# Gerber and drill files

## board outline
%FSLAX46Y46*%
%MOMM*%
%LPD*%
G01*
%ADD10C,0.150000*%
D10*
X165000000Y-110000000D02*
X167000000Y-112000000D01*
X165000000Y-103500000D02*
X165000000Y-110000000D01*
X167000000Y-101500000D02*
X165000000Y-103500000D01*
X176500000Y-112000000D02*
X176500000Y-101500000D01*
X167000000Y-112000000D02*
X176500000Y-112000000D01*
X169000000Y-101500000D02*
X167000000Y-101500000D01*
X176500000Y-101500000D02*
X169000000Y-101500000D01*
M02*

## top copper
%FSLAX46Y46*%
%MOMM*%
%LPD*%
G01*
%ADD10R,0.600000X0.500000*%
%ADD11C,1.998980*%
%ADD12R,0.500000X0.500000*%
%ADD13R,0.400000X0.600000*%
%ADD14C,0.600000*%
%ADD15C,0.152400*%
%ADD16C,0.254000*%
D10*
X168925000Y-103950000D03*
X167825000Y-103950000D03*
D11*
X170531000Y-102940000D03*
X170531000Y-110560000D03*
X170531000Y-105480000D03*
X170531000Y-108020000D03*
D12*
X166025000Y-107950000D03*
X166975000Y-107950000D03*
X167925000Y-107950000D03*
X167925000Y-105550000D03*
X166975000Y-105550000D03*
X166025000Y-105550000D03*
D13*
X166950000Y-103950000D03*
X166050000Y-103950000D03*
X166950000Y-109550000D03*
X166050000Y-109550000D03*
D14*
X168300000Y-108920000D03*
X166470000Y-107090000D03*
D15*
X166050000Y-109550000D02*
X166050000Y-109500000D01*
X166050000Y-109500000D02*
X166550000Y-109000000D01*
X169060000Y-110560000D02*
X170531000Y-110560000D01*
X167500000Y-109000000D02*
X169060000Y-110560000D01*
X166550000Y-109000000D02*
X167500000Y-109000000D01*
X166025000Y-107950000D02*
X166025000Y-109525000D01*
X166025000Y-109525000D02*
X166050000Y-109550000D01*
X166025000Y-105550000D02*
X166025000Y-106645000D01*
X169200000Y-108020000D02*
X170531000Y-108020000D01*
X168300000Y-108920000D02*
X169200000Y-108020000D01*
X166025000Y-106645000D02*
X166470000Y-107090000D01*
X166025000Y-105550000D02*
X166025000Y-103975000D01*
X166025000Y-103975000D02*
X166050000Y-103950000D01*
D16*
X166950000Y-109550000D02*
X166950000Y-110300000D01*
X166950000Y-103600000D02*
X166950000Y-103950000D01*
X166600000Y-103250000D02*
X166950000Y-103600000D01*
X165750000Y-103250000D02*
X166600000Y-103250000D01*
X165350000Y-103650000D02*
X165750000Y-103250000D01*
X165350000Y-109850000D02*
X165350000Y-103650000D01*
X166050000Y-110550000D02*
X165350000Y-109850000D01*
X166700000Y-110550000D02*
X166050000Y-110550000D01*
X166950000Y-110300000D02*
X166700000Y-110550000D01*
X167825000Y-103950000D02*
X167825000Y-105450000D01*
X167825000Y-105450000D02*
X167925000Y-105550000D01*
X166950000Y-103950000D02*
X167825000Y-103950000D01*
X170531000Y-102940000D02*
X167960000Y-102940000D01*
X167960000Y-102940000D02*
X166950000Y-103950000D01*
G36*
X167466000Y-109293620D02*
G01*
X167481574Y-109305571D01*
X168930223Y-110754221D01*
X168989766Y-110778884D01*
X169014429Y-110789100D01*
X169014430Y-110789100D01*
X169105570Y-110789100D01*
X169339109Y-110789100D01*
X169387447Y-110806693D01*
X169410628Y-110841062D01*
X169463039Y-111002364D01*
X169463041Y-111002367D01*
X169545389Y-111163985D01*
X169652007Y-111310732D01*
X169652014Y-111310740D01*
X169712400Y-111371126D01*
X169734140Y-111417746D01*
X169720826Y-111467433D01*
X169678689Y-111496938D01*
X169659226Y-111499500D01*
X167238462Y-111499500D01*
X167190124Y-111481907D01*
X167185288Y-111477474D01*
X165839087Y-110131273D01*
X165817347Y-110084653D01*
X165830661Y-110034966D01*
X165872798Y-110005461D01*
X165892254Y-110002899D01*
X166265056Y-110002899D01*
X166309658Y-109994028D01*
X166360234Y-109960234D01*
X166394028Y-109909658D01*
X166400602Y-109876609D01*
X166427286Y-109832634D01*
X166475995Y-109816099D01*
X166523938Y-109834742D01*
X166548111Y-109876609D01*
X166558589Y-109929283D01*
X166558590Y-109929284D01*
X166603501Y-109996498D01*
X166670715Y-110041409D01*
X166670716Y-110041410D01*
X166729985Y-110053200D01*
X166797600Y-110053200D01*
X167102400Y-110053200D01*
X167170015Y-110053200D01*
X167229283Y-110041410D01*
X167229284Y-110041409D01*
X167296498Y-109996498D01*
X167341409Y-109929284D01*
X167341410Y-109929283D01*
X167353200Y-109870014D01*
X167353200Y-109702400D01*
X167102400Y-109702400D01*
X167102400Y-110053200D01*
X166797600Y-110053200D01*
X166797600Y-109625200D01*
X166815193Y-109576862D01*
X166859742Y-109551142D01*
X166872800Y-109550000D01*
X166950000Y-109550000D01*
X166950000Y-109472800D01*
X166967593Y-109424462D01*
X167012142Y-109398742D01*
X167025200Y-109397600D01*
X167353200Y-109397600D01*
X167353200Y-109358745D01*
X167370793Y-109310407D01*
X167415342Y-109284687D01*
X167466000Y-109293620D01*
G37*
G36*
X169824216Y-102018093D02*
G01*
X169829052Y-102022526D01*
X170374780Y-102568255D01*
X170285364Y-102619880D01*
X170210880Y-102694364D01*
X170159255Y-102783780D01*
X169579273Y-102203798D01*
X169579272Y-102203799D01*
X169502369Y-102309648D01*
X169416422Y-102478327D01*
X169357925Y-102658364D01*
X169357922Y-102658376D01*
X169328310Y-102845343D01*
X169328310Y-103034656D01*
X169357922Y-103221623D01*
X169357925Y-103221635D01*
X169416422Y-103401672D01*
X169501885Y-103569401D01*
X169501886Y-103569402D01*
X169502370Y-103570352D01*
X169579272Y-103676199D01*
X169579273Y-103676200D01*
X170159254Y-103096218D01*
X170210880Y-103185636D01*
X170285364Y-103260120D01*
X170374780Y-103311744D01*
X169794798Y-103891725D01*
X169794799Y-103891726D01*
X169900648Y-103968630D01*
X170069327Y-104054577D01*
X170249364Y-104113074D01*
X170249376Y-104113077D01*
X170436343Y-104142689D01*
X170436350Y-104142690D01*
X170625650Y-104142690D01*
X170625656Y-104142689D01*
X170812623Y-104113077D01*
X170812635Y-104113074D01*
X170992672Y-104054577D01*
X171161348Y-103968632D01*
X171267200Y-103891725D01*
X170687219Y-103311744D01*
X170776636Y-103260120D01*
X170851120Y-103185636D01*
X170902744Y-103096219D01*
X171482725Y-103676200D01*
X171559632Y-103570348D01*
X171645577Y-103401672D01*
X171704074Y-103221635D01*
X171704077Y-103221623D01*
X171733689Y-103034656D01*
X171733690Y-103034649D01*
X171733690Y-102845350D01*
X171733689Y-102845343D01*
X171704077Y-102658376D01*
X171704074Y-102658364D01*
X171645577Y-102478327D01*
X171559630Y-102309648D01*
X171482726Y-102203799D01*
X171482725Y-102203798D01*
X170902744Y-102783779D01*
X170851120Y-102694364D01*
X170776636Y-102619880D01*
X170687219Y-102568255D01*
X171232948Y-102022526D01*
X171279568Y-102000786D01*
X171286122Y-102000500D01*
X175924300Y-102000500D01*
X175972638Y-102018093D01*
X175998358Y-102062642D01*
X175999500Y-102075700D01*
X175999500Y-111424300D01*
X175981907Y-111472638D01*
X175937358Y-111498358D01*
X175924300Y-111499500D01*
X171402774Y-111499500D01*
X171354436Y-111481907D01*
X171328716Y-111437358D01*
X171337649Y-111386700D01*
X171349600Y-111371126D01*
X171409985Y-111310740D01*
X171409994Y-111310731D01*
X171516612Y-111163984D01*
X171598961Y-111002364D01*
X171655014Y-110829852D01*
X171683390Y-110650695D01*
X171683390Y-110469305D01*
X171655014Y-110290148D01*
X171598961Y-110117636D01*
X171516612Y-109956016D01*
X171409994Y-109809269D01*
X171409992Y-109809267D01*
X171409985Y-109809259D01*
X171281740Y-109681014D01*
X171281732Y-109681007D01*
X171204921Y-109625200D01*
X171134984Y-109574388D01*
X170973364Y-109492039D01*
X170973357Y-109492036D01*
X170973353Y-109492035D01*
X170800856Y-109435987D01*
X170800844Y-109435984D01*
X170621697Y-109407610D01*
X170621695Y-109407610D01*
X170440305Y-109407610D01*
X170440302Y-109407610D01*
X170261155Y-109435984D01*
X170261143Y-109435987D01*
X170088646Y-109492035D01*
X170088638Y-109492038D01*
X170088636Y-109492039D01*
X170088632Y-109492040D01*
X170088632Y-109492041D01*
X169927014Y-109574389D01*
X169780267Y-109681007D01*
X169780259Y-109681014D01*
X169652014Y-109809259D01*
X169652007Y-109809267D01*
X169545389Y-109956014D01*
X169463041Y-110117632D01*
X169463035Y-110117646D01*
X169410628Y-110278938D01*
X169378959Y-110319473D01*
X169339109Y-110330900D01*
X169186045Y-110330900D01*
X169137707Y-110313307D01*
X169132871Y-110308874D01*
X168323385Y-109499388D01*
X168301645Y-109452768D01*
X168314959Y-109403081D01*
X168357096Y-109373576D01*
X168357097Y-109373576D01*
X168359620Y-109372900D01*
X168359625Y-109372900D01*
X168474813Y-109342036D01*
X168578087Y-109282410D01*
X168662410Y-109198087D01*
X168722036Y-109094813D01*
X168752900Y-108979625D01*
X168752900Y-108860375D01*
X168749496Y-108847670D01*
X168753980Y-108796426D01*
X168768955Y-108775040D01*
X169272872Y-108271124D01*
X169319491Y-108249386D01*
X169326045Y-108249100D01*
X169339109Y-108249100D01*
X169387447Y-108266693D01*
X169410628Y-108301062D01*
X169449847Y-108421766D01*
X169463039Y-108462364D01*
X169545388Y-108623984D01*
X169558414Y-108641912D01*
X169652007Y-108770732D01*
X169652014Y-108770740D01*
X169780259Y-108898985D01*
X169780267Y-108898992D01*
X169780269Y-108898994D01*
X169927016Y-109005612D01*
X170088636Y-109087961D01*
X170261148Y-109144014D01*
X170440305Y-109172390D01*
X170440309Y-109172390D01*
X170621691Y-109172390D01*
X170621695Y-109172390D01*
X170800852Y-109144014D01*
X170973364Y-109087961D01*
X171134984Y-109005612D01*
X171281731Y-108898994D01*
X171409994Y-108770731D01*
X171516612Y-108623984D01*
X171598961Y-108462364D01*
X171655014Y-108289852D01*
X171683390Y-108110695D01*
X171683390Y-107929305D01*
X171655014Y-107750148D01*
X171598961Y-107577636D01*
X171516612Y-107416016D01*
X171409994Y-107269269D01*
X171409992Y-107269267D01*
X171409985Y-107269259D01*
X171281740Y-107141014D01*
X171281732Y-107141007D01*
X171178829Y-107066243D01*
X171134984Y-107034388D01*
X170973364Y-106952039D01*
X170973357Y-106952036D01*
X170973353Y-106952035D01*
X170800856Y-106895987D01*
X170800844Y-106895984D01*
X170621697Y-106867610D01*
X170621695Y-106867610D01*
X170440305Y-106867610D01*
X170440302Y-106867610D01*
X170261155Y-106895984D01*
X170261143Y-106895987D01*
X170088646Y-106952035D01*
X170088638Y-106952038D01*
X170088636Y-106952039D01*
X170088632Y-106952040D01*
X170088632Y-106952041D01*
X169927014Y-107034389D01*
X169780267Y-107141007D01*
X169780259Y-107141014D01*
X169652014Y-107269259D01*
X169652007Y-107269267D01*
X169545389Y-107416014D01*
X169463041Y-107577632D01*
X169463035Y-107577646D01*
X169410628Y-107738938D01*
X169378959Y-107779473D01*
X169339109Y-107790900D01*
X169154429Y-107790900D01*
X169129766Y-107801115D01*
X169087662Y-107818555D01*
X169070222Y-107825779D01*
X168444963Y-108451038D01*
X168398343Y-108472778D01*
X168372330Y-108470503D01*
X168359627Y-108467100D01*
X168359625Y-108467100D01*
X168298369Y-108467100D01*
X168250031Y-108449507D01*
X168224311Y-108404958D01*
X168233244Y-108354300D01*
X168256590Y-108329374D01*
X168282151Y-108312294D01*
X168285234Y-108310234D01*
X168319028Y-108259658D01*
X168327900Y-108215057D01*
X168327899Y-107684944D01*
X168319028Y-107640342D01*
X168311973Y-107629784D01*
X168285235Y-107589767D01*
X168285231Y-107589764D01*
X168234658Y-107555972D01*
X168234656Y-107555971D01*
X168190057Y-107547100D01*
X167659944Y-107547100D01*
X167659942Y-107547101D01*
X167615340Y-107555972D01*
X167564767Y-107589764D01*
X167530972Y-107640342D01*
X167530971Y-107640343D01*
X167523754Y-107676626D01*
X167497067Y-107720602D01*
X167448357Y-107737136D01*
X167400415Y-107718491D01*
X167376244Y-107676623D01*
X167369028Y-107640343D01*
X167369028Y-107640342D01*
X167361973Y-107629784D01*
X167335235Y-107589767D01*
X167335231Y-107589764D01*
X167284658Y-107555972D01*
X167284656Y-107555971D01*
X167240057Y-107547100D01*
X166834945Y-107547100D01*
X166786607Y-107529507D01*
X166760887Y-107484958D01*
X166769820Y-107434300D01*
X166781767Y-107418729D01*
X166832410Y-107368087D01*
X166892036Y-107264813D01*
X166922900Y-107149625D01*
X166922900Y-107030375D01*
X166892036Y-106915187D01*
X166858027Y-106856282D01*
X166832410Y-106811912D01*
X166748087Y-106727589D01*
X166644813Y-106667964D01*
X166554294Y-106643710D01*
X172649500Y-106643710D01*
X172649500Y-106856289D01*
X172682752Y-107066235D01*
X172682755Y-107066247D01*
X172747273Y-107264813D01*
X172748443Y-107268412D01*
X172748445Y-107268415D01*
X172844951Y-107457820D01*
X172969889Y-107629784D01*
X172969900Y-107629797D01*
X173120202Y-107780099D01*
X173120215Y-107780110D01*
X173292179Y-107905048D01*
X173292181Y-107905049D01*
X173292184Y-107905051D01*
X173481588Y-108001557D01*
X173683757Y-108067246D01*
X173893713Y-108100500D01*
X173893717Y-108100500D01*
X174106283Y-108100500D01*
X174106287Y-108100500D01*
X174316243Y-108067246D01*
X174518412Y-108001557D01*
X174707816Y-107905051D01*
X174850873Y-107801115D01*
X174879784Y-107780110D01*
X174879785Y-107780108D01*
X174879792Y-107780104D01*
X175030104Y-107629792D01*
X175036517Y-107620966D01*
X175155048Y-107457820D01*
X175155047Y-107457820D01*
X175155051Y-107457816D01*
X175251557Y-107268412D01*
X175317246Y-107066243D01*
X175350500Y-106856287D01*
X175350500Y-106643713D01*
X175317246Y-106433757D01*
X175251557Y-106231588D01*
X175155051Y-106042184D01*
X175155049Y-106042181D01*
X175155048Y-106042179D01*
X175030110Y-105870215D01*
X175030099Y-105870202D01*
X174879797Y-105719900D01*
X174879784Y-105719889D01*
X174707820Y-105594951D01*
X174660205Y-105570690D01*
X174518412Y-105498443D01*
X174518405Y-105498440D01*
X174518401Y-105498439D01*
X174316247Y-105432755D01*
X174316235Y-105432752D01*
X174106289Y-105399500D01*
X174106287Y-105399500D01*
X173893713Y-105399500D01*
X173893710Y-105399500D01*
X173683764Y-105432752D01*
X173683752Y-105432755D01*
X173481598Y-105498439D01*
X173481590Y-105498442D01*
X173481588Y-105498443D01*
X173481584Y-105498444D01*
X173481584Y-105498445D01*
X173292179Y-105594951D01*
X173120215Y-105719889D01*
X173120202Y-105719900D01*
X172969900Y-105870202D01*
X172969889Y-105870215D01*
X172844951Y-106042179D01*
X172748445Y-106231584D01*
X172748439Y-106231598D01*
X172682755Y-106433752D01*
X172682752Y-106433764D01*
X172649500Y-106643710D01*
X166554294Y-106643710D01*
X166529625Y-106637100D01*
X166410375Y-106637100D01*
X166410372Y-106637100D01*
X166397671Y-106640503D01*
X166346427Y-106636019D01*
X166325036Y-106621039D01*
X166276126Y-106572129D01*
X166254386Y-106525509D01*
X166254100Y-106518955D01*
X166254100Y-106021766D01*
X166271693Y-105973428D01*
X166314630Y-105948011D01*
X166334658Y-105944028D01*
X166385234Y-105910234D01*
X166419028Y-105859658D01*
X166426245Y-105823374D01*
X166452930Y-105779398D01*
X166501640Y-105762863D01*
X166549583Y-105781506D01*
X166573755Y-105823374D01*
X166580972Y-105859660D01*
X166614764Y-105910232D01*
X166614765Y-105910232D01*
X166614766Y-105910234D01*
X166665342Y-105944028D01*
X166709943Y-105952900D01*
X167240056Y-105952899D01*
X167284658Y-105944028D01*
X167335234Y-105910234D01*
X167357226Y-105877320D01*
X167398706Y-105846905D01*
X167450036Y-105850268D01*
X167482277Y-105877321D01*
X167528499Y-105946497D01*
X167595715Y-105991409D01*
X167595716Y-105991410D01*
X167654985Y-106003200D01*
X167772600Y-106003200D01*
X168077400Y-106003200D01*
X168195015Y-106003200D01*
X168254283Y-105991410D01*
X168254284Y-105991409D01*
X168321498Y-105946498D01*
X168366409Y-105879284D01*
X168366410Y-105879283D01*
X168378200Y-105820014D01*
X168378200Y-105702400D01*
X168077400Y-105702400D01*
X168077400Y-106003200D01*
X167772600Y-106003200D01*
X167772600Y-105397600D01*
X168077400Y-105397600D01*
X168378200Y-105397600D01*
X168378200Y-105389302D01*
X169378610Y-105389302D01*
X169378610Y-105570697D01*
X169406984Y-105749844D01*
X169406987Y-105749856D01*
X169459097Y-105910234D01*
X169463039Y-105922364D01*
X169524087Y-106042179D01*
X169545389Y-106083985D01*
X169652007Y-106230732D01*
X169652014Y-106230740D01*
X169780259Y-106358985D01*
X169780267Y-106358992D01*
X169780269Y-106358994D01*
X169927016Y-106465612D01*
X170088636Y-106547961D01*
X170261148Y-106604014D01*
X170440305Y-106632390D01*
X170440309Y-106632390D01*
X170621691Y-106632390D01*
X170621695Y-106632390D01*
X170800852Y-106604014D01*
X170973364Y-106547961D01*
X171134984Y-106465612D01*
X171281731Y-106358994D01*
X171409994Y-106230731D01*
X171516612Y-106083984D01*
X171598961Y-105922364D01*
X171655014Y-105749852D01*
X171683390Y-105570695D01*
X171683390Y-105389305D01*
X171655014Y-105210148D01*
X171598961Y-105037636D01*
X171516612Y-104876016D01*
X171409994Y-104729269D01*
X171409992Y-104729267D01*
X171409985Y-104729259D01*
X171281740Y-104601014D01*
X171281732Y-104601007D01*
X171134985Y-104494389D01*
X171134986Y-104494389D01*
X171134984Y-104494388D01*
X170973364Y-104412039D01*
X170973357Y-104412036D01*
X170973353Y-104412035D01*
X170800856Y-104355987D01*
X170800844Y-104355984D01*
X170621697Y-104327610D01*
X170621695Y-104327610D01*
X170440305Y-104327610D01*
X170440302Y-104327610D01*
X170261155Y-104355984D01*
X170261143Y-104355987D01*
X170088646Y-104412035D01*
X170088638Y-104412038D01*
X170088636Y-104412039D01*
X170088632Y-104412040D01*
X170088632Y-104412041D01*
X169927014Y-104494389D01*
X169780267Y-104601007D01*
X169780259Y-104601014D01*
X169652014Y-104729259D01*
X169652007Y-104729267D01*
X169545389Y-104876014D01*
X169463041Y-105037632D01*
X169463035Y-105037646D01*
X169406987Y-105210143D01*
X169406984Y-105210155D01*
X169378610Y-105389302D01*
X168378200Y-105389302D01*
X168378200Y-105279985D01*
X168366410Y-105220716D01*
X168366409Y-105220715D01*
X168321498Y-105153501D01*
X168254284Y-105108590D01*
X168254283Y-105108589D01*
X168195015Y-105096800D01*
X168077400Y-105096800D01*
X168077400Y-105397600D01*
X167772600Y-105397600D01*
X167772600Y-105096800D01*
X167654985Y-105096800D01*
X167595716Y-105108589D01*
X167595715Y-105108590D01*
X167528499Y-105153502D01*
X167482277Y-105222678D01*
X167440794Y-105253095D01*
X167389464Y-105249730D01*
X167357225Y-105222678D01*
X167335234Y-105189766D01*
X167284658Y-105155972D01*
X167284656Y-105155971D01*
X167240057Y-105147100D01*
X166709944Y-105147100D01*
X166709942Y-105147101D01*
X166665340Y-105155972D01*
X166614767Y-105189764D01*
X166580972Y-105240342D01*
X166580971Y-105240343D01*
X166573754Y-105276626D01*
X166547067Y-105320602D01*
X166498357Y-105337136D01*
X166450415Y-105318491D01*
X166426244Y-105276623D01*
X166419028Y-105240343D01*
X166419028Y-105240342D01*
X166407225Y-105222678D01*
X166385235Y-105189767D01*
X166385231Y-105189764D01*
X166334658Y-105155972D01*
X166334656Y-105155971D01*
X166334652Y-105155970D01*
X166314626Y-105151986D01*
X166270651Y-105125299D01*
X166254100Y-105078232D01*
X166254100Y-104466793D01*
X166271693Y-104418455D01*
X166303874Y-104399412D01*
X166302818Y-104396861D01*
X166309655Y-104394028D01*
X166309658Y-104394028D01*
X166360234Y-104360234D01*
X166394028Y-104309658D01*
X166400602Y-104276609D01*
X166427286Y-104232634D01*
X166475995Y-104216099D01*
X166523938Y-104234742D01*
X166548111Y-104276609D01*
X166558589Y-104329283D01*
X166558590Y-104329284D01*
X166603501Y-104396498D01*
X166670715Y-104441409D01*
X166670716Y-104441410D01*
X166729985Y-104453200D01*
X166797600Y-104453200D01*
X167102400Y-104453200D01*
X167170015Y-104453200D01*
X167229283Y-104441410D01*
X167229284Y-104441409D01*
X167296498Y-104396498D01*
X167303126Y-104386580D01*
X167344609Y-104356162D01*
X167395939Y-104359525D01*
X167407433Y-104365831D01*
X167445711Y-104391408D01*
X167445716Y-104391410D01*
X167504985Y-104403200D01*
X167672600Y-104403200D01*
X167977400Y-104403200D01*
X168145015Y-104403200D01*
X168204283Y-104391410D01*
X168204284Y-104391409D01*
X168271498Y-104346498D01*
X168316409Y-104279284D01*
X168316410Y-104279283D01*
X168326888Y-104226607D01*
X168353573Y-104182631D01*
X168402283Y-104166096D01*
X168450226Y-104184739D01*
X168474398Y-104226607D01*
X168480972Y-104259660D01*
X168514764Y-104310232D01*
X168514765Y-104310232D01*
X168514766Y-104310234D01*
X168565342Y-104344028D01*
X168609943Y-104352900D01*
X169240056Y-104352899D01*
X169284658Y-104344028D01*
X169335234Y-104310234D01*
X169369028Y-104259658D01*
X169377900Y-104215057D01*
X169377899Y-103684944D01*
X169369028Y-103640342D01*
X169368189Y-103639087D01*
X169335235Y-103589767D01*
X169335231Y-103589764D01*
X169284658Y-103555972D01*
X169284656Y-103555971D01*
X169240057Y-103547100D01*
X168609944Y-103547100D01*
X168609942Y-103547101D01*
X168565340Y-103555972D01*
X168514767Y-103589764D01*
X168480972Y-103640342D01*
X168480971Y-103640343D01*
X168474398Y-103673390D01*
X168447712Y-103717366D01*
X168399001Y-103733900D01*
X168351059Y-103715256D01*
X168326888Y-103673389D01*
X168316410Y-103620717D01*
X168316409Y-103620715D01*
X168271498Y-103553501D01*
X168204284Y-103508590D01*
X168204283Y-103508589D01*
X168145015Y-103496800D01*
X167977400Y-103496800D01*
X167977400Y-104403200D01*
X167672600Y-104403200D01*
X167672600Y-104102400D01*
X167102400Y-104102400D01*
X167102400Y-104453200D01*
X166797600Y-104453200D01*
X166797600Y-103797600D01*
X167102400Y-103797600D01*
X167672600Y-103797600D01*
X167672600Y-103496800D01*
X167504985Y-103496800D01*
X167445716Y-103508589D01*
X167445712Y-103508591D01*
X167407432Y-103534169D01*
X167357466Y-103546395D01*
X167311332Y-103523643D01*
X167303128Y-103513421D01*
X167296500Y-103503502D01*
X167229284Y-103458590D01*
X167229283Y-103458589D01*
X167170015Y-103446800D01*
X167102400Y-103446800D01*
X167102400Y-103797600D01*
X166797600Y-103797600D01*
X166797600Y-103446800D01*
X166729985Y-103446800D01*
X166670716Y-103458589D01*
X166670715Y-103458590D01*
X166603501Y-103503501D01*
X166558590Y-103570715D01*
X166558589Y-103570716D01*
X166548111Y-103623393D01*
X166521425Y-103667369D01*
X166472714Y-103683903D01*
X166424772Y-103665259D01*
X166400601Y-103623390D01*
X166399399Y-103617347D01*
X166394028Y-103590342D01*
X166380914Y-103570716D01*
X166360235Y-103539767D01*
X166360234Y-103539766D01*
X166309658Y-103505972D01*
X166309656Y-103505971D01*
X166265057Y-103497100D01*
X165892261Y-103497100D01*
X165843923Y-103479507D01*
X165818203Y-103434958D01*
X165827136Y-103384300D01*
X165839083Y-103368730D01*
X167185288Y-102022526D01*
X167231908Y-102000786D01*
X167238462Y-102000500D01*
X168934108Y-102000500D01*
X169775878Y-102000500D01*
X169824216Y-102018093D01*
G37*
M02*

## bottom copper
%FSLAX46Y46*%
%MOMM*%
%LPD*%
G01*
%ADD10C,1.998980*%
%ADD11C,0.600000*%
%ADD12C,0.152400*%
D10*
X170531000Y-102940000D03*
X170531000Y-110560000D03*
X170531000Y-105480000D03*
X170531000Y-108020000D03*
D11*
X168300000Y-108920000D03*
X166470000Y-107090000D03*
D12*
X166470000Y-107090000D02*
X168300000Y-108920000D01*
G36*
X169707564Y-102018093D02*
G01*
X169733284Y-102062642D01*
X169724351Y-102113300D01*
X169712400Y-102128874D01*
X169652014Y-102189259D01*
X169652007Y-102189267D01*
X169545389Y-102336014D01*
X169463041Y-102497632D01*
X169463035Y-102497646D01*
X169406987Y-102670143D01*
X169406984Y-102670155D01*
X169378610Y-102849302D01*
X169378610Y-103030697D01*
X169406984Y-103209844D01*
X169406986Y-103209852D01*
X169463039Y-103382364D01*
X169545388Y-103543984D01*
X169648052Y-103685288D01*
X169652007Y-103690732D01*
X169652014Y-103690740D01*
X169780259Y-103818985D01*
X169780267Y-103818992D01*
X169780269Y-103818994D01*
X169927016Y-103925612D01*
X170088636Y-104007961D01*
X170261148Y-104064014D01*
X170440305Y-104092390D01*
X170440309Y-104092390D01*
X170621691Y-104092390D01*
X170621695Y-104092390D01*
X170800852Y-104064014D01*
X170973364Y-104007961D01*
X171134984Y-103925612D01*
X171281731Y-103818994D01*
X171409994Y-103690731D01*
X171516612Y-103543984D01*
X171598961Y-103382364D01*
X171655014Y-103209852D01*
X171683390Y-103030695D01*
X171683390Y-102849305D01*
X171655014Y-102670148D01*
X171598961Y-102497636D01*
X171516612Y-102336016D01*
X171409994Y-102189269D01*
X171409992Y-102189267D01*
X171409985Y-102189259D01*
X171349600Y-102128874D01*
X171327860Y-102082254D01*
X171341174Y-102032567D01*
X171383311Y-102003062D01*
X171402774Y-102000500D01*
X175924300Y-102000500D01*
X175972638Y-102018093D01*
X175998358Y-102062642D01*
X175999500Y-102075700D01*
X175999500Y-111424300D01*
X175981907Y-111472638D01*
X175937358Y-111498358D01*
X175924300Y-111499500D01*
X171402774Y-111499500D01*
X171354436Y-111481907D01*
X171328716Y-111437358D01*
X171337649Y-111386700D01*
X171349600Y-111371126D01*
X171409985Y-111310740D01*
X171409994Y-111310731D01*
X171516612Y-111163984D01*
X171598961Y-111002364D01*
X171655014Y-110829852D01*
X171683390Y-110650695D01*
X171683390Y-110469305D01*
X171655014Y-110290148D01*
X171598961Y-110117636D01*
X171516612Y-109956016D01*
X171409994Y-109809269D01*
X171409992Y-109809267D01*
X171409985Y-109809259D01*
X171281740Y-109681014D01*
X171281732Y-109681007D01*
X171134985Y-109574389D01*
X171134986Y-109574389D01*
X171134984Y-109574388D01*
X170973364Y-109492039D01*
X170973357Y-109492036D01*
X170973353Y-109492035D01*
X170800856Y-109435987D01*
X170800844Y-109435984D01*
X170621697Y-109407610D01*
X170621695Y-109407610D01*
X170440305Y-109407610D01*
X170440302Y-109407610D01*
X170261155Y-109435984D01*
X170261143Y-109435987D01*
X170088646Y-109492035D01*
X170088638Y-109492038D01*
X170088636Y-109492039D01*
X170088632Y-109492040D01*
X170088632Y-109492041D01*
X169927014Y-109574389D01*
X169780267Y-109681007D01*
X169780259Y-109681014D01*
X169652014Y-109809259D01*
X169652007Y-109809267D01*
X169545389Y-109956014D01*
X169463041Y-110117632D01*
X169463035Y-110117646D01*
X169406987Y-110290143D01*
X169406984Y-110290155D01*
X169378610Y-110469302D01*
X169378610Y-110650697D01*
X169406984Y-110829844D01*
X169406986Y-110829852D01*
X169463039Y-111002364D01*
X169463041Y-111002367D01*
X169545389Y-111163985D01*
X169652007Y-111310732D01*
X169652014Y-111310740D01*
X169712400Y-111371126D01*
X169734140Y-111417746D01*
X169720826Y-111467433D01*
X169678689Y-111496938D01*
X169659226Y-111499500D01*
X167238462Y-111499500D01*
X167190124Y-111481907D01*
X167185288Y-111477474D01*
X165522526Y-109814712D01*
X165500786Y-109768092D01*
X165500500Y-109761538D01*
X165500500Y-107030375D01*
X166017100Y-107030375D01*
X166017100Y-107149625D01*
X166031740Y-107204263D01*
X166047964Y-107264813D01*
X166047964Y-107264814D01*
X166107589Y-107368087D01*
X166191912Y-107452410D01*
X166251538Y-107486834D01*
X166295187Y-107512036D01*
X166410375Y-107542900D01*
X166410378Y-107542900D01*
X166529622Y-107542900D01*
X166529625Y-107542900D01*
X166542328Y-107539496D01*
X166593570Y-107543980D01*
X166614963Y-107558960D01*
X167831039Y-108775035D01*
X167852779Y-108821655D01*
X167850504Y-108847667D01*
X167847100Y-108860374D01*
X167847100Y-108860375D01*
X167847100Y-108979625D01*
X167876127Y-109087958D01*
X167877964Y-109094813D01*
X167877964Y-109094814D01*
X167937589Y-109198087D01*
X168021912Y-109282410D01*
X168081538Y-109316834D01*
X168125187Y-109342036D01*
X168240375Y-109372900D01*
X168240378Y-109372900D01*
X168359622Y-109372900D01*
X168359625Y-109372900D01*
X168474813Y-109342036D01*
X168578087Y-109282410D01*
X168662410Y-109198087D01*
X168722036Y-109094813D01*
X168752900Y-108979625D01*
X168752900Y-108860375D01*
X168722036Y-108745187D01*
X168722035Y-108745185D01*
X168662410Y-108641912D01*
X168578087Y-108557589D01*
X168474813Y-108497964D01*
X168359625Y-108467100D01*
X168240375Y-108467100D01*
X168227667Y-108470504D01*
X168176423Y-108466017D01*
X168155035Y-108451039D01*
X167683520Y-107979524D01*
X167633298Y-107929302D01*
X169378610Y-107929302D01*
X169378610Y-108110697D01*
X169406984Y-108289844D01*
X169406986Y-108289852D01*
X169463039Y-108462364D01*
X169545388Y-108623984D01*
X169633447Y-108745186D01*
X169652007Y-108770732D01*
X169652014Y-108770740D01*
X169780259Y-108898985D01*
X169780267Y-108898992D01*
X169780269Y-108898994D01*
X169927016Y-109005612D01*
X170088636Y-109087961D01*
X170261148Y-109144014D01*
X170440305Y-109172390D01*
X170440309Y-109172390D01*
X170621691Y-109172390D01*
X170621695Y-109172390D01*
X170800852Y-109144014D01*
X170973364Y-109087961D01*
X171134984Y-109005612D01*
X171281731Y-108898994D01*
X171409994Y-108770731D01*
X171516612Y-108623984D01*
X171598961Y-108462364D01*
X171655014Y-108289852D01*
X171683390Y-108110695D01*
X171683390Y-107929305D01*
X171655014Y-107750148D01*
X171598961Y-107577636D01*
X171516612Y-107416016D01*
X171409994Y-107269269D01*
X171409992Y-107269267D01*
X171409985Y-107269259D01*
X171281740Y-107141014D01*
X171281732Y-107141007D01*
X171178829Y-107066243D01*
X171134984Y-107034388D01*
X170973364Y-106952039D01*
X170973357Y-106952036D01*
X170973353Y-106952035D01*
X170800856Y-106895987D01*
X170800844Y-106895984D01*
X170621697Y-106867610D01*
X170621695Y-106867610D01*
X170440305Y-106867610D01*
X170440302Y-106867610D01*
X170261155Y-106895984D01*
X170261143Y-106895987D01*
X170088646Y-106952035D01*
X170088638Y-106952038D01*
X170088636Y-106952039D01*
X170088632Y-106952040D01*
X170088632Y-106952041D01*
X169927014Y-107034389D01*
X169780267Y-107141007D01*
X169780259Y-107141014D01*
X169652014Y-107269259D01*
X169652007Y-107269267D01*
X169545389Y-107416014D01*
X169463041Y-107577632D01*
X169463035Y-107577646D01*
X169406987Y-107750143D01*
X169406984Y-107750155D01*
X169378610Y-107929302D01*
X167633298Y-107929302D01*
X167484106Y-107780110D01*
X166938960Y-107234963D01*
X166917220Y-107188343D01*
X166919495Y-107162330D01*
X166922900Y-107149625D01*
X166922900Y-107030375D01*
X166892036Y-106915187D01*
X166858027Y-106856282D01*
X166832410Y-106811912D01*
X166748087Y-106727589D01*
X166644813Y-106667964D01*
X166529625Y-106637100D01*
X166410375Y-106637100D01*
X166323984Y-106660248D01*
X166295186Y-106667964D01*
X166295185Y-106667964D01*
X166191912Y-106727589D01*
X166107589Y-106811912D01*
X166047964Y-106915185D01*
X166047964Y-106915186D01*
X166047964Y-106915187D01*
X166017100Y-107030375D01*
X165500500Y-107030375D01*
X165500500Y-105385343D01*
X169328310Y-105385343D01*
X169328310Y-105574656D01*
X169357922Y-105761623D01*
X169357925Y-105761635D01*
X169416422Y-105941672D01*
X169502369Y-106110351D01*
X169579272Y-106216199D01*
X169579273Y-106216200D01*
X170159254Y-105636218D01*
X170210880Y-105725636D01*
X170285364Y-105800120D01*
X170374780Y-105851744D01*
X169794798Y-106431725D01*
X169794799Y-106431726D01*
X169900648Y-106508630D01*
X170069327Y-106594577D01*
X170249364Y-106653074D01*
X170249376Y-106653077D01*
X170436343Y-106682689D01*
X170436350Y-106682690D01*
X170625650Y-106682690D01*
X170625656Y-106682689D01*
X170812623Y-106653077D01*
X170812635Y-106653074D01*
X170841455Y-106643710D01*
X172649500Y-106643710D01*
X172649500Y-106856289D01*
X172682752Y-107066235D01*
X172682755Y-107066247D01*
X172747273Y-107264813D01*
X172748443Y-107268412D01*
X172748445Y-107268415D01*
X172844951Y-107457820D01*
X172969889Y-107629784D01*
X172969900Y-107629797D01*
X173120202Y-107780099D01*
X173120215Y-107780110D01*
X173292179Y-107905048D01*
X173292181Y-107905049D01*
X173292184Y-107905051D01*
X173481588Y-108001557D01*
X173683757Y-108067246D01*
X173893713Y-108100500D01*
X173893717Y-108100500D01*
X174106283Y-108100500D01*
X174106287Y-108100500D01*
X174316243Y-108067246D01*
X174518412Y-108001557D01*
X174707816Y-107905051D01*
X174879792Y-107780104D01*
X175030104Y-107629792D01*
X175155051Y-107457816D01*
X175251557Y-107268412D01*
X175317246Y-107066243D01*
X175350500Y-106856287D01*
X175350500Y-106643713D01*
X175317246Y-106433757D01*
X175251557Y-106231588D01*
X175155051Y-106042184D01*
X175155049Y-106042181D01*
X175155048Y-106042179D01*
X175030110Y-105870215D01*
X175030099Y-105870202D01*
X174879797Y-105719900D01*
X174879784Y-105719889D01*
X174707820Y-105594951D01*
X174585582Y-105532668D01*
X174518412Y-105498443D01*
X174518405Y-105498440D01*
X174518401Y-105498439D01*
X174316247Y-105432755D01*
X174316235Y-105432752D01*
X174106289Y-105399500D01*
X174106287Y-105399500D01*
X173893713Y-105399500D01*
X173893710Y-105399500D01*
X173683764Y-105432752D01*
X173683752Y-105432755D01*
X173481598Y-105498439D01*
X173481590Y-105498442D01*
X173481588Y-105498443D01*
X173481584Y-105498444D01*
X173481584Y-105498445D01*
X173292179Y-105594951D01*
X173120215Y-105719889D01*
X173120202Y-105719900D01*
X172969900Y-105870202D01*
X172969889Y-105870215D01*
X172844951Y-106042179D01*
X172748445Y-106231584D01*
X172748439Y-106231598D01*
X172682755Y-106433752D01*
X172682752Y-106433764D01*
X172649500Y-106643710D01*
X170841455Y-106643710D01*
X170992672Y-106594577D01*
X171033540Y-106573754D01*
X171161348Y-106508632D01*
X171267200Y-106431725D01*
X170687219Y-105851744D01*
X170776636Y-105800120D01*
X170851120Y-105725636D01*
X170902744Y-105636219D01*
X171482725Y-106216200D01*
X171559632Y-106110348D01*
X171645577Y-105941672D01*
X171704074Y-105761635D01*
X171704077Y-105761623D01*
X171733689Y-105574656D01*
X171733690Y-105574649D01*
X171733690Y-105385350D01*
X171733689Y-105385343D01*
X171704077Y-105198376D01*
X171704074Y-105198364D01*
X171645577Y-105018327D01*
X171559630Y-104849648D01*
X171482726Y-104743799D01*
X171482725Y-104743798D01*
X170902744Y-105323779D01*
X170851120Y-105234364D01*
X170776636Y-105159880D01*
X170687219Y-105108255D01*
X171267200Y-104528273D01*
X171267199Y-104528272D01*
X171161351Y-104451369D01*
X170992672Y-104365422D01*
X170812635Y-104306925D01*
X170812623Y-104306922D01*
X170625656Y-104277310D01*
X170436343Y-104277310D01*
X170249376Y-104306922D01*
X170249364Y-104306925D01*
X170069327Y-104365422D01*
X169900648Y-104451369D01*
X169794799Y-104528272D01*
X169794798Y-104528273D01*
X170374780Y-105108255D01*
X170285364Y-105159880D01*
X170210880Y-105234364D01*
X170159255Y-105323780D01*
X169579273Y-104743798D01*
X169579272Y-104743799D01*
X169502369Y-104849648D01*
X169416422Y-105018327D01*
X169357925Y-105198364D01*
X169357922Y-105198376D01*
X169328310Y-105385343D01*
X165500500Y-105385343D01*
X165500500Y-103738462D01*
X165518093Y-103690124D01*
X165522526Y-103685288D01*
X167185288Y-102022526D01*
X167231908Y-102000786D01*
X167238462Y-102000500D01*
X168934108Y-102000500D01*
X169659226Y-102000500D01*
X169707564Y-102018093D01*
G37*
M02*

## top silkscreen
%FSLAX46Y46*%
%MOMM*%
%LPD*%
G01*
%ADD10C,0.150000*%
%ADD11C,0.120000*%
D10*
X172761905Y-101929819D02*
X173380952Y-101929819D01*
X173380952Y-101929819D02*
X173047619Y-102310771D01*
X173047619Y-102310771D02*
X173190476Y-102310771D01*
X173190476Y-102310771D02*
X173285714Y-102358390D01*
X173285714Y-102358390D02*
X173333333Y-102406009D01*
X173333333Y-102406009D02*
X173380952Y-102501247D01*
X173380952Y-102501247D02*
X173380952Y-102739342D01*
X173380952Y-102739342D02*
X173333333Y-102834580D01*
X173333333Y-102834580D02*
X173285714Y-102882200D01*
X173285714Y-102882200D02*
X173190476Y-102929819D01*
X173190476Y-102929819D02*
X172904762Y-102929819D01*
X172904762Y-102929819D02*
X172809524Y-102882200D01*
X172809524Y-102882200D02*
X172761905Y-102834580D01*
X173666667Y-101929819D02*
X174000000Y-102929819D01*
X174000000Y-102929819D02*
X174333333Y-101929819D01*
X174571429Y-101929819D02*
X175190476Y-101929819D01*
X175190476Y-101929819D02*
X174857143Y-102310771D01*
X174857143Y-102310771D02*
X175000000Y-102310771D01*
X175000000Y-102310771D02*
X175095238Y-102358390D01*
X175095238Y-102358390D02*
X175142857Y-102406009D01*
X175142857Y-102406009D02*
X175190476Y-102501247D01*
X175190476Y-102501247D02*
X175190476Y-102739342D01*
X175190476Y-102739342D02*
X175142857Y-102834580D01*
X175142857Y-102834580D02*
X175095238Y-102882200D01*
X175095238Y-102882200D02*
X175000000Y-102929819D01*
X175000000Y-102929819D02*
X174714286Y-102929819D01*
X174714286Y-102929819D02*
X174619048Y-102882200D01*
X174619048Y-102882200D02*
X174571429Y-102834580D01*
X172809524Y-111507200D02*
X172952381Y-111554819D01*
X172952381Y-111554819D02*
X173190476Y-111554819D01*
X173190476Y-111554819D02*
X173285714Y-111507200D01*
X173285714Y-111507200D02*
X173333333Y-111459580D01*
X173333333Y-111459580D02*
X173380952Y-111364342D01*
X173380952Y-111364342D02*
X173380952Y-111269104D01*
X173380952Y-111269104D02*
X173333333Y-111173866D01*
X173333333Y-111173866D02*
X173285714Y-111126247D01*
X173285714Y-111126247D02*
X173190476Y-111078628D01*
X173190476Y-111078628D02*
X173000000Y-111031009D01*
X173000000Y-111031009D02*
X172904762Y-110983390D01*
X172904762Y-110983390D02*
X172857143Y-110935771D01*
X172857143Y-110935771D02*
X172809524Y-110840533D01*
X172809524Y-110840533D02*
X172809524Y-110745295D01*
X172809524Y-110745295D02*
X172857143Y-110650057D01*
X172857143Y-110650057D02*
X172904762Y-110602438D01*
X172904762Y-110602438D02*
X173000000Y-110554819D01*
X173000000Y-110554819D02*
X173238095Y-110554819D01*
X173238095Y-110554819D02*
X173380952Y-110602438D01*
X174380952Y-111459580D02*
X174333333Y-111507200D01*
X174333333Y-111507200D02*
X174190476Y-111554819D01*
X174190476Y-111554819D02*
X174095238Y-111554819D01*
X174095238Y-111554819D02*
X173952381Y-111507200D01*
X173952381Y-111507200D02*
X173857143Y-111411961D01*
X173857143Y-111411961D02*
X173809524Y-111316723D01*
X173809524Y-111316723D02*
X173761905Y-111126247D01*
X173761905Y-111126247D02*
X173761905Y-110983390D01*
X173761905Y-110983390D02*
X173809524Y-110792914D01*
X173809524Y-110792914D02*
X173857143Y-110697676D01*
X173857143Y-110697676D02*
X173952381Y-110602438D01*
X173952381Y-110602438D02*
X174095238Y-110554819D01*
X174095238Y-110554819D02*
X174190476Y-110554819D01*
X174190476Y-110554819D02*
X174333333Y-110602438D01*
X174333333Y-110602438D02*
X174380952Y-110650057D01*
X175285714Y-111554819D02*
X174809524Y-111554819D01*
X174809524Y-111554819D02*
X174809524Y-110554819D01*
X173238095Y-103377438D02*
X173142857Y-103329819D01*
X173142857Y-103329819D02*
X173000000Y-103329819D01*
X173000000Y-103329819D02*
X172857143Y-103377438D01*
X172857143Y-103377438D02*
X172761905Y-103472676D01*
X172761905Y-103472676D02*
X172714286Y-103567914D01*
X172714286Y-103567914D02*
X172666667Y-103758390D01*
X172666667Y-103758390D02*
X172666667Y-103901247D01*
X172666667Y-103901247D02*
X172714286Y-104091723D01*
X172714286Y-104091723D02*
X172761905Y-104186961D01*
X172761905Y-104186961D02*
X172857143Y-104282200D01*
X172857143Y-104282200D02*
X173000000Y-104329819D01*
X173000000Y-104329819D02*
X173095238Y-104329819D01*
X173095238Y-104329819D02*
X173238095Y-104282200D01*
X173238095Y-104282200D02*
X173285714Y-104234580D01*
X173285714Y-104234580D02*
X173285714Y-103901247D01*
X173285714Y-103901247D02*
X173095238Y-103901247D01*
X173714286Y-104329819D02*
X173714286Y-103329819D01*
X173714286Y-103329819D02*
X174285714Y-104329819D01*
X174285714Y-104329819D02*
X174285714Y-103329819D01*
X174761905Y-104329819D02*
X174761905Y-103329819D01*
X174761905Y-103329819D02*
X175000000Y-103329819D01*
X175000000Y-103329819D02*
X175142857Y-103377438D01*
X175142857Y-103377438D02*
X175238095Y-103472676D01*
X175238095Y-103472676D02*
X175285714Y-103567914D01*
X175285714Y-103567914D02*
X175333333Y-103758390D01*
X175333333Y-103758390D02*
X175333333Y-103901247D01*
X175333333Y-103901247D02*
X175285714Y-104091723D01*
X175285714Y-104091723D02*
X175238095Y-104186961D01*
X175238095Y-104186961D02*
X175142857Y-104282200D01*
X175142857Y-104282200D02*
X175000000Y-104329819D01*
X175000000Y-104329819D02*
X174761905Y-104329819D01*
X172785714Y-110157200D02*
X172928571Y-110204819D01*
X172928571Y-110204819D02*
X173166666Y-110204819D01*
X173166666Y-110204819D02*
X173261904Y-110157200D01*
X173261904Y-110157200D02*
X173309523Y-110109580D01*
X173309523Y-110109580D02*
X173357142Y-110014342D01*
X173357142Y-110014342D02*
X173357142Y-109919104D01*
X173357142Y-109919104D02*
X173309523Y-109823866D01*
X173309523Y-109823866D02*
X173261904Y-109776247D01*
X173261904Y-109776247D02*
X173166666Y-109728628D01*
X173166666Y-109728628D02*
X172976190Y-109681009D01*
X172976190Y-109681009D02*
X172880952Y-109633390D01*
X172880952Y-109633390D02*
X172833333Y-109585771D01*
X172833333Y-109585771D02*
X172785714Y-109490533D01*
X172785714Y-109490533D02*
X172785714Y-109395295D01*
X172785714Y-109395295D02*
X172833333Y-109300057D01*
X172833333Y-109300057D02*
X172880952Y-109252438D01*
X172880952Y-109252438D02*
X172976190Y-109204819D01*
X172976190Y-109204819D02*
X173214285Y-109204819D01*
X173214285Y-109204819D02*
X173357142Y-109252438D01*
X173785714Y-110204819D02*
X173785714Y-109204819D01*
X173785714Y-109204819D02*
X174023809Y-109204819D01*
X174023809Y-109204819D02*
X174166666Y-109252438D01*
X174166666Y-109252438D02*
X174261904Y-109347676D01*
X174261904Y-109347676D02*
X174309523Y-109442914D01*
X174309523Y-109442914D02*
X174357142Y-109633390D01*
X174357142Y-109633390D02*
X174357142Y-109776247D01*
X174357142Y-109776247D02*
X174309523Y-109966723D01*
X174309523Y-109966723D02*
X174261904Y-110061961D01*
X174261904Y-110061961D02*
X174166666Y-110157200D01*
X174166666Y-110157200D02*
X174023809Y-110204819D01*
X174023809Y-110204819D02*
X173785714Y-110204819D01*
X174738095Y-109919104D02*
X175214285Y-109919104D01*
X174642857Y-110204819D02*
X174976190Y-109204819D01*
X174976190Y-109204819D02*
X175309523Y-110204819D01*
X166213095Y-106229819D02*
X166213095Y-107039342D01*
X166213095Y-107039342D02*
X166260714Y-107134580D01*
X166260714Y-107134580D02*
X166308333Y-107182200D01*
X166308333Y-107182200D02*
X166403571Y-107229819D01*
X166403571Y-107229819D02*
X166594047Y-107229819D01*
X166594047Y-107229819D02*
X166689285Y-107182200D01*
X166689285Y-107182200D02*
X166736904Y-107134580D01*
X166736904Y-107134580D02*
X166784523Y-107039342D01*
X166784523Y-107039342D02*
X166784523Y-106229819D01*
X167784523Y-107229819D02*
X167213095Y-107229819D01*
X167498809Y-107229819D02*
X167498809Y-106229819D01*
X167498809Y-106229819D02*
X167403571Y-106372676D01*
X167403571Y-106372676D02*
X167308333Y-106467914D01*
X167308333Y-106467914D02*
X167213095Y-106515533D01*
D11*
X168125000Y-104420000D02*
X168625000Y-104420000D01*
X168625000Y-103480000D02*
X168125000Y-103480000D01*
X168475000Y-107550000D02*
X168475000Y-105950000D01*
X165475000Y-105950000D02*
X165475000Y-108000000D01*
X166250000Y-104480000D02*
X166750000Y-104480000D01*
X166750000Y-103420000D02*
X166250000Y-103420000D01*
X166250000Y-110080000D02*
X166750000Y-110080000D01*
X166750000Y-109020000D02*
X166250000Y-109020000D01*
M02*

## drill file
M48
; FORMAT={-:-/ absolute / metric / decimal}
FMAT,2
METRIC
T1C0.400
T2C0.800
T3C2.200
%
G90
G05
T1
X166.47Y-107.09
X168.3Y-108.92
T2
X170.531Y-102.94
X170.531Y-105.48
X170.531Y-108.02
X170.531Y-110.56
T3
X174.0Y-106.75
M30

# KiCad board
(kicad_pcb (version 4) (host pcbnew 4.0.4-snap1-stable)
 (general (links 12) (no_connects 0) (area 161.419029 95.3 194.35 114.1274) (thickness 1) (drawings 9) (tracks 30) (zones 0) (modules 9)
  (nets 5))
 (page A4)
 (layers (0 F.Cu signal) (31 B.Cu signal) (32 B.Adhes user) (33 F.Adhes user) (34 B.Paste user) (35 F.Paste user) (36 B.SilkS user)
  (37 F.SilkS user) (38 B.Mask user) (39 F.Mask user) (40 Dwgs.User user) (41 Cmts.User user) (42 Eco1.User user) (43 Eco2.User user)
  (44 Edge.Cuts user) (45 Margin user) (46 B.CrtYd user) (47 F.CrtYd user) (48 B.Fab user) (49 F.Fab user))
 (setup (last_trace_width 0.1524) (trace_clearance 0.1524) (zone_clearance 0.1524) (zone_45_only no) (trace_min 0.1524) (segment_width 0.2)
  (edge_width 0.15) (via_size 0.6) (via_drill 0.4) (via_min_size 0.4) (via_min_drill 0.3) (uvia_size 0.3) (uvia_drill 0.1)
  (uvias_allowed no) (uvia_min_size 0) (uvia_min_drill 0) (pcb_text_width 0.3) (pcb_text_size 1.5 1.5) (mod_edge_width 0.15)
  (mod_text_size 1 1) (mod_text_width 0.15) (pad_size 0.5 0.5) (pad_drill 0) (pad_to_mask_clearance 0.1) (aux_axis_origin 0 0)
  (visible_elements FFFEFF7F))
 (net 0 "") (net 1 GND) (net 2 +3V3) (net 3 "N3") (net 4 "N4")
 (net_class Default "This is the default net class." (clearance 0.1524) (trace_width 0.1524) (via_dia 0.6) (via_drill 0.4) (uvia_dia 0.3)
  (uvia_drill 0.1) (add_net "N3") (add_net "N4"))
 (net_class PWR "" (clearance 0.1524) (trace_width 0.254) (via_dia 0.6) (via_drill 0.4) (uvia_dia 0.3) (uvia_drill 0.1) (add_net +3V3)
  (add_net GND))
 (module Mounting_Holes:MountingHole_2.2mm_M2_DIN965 (layer F.Cu) (at 174 106.75)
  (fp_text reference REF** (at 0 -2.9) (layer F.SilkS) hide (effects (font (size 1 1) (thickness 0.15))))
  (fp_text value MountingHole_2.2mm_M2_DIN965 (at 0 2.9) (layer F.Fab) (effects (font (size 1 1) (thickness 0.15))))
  (pad 1 np_thru_hole circle (at 0 0) (size 2.2 2.2) (drill 2.2) (layers *.Cu *.Mask)))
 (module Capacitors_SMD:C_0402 (layer F.Cu) (at 168.375 103.95 180)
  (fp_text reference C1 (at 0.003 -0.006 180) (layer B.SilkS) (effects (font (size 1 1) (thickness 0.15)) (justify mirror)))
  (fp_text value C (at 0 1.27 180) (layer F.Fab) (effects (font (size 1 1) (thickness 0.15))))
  (fp_line (start 0.25 -0.47) (end -0.25 -0.47) (layer F.SilkS) (width 0.12))
  (fp_line (start -0.25 0.47) (end 0.25 0.47) (layer F.SilkS) (width 0.12))
  (pad 1 smd rect (at -0.55 0 180) (size 0.6 0.5) (layers F.Cu F.Paste F.Mask) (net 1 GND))
  (pad 2 smd rect (at 0.55 0 180) (size 0.6 0.5) (layers F.Cu F.Paste F.Mask) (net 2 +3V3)))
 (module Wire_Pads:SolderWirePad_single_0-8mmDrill (layer F.Cu) (at 170.531 102.94)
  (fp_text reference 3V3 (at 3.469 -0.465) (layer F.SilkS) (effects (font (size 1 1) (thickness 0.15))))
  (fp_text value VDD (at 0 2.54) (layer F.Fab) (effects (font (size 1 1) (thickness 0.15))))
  (pad 1 thru_hole circle (at 0 0) (size 1.99898 1.99898) (drill 0.8001) (layers *.Cu *.Mask) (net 2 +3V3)))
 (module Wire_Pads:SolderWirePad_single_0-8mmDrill (layer F.Cu) (at 170.531 110.56)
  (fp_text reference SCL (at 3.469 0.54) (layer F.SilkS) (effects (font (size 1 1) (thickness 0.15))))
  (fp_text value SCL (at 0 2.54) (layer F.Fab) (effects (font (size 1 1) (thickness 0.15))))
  (pad 1 thru_hole circle (at 0 0) (size 1.99898 1.99898) (drill 0.8001) (layers *.Cu *.Mask) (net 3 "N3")))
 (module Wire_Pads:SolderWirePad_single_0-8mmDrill (layer F.Cu) (at 170.531 105.48)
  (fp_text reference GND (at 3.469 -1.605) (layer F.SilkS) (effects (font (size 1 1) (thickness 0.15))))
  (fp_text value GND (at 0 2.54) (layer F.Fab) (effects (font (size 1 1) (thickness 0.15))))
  (pad 1 thru_hole circle (at 0 0) (size 1.99898 1.99898) (drill 0.8001) (layers *.Cu *.Mask) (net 1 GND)))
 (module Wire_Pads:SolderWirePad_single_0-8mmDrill (layer F.Cu) (at 170.531 108.02)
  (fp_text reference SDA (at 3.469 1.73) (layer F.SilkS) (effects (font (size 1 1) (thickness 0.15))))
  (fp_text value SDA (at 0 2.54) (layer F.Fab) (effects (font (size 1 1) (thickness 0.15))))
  (pad 1 thru_hole circle (at 0 0) (size 1.99898 1.99898) (drill 0.8001) (layers *.Cu *.Mask) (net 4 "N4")))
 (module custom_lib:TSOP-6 (layer F.Cu) (at 166.975 106.75 90)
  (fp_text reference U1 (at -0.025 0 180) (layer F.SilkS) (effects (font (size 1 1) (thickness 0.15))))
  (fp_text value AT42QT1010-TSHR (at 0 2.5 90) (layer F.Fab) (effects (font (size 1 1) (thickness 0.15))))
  (fp_line (start -0.8 1.5) (end 0.8 1.5) (layer F.SilkS) (width 0.12))
  (fp_line (start 0.8 -1.5) (end -1.25 -1.5) (layer F.SilkS) (width 0.12))
  (pad 1 smd rect (at -1.2 -0.95 90) (size 0.5 0.5) (layers F.Cu F.Paste F.Mask) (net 3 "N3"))
  (pad 2 smd rect (at -1.2 0 90) (size 0.5 0.5) (layers F.Cu F.Paste F.Mask) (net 1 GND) (zone_connect 2))
  (pad 3 smd rect (at -1.2 0.95 90) (size 0.5 0.5) (layers F.Cu F.Paste F.Mask) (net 1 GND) (zone_connect 2))
  (pad 4 smd rect (at 1.2 0.95 90) (size 0.5 0.5) (layers F.Cu F.Paste F.Mask) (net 2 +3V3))
  (pad 5 smd rect (at 1.2 0 90) (size 0.5 0.5) (layers F.Cu F.Paste F.Mask) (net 1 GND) (zone_connect 2))
  (pad 6 smd rect (at 1.2 -0.95 90) (size 0.5 0.5) (layers F.Cu F.Paste F.Mask) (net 4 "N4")))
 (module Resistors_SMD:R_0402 (layer F.Cu) (at 166.5 103.95 180)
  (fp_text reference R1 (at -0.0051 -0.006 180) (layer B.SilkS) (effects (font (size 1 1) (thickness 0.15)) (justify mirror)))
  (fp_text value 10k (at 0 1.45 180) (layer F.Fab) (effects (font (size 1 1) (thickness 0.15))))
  (fp_line (start 0.25 -0.53) (end -0.25 -0.53) (layer F.SilkS) (width 0.12))
  (fp_line (start -0.25 0.53) (end 0.25 0.53) (layer F.SilkS) (width 0.12))
  (pad 1 smd rect (at -0.45 0 180) (size 0.4 0.6) (layers F.Cu F.Paste F.Mask) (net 2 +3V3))
  (pad 2 smd rect (at 0.45 0 180) (size 0.4 0.6) (layers F.Cu F.Paste F.Mask) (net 4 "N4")))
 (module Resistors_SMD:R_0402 (layer F.Cu) (at 166.5 109.55 180)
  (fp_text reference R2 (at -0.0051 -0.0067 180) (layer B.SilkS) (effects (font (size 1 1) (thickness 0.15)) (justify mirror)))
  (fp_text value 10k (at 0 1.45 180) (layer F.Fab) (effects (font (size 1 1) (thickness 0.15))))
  (fp_line (start 0.25 -0.53) (end -0.25 -0.53) (layer F.SilkS) (width 0.12))
  (fp_line (start -0.25 0.53) (end 0.25 0.53) (layer F.SilkS) (width 0.12))
  (pad 1 smd rect (at -0.45 0 180) (size 0.4 0.6) (layers F.Cu F.Paste F.Mask) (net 2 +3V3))
  (pad 2 smd rect (at 0.45 0 180) (size 0.4 0.6) (layers F.Cu F.Paste F.Mask) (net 3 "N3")))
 (gr_line (start 165 110) (end 167 112) (angle 90) (layer Edge.Cuts) (width 0.15))
 (gr_line (start 165 103.5) (end 165 110) (angle 90) (layer Edge.Cuts) (width 0.15))
 (gr_line (start 167 101.5) (end 165 103.5) (angle 90) (layer Edge.Cuts) (width 0.15))
 (gr_line (start 176.5 112) (end 176.5 101.5) (angle 90) (layer Edge.Cuts) (width 0.15))
 (gr_line (start 167 112) (end 176.5 112) (angle 90) (layer Edge.Cuts) (width 0.15))
 (gr_line (start 169 101.5) (end 167 101.5) (angle 90) (layer Edge.Cuts) (width 0.15))
 (gr_line (start 176.5 101.5) (end 169 101.5) (angle 90) (layer Edge.Cuts) (width 0.15))
 (segment (start 166.05 109.55) (end 166.05 109.5) (width 0.1524) (layer F.Cu) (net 3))
 (segment (start 166.05 109.5) (end 166.55 109) (width 0.1524) (layer F.Cu) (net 3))
 (segment (start 169.06 110.56) (end 170.531 110.56) (width 0.1524) (layer F.Cu) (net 3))
 (segment (start 167.5 109) (end 169.06 110.56) (width 0.1524) (layer F.Cu) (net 3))
 (segment (start 166.55 109) (end 167.5 109) (width 0.1524) (layer F.Cu) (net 3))
 (segment (start 166.025 107.95) (end 166.025 109.525) (width 0.1524) (layer F.Cu) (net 3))
 (segment (start 166.025 109.525) (end 166.05 109.55) (width 0.1524) (layer F.Cu) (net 3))
 (segment (start 166.025 105.55) (end 166.025 106.645) (width 0.1524) (layer F.Cu) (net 4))
 (segment (start 169.2 108.02) (end 170.531 108.02) (width 0.1524) (layer F.Cu) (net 4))
 (segment (start 168.3 108.92) (end 169.2 108.02) (width 0.1524) (layer F.Cu) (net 4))
 (via (at 168.3 108.92) (size 0.6) (drill 0.4) (layers F.Cu B.Cu) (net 4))
 (segment (start 166.47 107.09) (end 168.3 108.92) (width 0.1524) (layer B.Cu) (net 4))
 (via (at 166.47 107.09) (size 0.6) (drill 0.4) (layers F.Cu B.Cu) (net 4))
 (segment (start 166.025 106.645) (end 166.47 107.09) (width 0.1524) (layer F.Cu) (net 4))
 (segment (start 166.025 105.55) (end 166.025 103.975) (width 0.1524) (layer F.Cu) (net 4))
 (segment (start 166.025 103.975) (end 166.05 103.95) (width 0.1524) (layer F.Cu) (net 4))
 (segment (start 166.95 109.55) (end 166.95 110.3) (width 0.254) (layer F.Cu) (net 2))
 (segment (start 166.95 103.6) (end 166.95 103.95) (width 0.254) (layer F.Cu) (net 2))
 (segment (start 166.6 103.25) (end 166.95 103.6) (width 0.254) (layer F.Cu) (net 2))
 (segment (start 165.75 103.25) (end 166.6 103.25) (width 0.254) (layer F.Cu) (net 2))
 (segment (start 165.35 103.65) (end 165.75 103.25) (width 0.254) (layer F.Cu) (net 2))
 (segment (start 165.35 109.85) (end 165.35 103.65) (width 0.254) (layer F.Cu) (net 2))
 (segment (start 166.05 110.55) (end 165.35 109.85) (width 0.254) (layer F.Cu) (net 2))
 (segment (start 166.7 110.55) (end 166.05 110.55) (width 0.254) (layer F.Cu) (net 2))
 (segment (start 166.95 110.3) (end 166.7 110.55) (width 0.254) (layer F.Cu) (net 2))
 (segment (start 167.825 103.95) (end 167.825 105.45) (width 0.254) (layer F.Cu) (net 2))
 (segment (start 167.825 105.45) (end 167.925 105.55) (width 0.254) (layer F.Cu) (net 2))
 (segment (start 166.95 103.95) (end 167.825 103.95) (width 0.254) (layer F.Cu) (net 2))
 (segment (start 170.531 102.94) (end 167.96 102.94) (width 0.254) (layer F.Cu) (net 2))
 (segment (start 167.96 102.94) (end 166.95 103.95) (width 0.254) (layer F.Cu) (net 2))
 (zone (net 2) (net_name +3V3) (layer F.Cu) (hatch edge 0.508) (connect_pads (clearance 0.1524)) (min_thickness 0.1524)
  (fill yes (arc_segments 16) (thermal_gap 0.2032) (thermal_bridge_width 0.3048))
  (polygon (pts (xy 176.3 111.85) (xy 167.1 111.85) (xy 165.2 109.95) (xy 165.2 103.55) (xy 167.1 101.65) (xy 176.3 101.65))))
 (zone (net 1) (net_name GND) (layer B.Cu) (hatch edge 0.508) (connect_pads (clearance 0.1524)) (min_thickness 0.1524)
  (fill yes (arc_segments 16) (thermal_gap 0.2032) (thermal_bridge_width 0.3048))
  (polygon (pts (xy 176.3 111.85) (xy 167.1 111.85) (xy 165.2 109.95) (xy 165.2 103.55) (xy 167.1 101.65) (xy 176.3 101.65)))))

